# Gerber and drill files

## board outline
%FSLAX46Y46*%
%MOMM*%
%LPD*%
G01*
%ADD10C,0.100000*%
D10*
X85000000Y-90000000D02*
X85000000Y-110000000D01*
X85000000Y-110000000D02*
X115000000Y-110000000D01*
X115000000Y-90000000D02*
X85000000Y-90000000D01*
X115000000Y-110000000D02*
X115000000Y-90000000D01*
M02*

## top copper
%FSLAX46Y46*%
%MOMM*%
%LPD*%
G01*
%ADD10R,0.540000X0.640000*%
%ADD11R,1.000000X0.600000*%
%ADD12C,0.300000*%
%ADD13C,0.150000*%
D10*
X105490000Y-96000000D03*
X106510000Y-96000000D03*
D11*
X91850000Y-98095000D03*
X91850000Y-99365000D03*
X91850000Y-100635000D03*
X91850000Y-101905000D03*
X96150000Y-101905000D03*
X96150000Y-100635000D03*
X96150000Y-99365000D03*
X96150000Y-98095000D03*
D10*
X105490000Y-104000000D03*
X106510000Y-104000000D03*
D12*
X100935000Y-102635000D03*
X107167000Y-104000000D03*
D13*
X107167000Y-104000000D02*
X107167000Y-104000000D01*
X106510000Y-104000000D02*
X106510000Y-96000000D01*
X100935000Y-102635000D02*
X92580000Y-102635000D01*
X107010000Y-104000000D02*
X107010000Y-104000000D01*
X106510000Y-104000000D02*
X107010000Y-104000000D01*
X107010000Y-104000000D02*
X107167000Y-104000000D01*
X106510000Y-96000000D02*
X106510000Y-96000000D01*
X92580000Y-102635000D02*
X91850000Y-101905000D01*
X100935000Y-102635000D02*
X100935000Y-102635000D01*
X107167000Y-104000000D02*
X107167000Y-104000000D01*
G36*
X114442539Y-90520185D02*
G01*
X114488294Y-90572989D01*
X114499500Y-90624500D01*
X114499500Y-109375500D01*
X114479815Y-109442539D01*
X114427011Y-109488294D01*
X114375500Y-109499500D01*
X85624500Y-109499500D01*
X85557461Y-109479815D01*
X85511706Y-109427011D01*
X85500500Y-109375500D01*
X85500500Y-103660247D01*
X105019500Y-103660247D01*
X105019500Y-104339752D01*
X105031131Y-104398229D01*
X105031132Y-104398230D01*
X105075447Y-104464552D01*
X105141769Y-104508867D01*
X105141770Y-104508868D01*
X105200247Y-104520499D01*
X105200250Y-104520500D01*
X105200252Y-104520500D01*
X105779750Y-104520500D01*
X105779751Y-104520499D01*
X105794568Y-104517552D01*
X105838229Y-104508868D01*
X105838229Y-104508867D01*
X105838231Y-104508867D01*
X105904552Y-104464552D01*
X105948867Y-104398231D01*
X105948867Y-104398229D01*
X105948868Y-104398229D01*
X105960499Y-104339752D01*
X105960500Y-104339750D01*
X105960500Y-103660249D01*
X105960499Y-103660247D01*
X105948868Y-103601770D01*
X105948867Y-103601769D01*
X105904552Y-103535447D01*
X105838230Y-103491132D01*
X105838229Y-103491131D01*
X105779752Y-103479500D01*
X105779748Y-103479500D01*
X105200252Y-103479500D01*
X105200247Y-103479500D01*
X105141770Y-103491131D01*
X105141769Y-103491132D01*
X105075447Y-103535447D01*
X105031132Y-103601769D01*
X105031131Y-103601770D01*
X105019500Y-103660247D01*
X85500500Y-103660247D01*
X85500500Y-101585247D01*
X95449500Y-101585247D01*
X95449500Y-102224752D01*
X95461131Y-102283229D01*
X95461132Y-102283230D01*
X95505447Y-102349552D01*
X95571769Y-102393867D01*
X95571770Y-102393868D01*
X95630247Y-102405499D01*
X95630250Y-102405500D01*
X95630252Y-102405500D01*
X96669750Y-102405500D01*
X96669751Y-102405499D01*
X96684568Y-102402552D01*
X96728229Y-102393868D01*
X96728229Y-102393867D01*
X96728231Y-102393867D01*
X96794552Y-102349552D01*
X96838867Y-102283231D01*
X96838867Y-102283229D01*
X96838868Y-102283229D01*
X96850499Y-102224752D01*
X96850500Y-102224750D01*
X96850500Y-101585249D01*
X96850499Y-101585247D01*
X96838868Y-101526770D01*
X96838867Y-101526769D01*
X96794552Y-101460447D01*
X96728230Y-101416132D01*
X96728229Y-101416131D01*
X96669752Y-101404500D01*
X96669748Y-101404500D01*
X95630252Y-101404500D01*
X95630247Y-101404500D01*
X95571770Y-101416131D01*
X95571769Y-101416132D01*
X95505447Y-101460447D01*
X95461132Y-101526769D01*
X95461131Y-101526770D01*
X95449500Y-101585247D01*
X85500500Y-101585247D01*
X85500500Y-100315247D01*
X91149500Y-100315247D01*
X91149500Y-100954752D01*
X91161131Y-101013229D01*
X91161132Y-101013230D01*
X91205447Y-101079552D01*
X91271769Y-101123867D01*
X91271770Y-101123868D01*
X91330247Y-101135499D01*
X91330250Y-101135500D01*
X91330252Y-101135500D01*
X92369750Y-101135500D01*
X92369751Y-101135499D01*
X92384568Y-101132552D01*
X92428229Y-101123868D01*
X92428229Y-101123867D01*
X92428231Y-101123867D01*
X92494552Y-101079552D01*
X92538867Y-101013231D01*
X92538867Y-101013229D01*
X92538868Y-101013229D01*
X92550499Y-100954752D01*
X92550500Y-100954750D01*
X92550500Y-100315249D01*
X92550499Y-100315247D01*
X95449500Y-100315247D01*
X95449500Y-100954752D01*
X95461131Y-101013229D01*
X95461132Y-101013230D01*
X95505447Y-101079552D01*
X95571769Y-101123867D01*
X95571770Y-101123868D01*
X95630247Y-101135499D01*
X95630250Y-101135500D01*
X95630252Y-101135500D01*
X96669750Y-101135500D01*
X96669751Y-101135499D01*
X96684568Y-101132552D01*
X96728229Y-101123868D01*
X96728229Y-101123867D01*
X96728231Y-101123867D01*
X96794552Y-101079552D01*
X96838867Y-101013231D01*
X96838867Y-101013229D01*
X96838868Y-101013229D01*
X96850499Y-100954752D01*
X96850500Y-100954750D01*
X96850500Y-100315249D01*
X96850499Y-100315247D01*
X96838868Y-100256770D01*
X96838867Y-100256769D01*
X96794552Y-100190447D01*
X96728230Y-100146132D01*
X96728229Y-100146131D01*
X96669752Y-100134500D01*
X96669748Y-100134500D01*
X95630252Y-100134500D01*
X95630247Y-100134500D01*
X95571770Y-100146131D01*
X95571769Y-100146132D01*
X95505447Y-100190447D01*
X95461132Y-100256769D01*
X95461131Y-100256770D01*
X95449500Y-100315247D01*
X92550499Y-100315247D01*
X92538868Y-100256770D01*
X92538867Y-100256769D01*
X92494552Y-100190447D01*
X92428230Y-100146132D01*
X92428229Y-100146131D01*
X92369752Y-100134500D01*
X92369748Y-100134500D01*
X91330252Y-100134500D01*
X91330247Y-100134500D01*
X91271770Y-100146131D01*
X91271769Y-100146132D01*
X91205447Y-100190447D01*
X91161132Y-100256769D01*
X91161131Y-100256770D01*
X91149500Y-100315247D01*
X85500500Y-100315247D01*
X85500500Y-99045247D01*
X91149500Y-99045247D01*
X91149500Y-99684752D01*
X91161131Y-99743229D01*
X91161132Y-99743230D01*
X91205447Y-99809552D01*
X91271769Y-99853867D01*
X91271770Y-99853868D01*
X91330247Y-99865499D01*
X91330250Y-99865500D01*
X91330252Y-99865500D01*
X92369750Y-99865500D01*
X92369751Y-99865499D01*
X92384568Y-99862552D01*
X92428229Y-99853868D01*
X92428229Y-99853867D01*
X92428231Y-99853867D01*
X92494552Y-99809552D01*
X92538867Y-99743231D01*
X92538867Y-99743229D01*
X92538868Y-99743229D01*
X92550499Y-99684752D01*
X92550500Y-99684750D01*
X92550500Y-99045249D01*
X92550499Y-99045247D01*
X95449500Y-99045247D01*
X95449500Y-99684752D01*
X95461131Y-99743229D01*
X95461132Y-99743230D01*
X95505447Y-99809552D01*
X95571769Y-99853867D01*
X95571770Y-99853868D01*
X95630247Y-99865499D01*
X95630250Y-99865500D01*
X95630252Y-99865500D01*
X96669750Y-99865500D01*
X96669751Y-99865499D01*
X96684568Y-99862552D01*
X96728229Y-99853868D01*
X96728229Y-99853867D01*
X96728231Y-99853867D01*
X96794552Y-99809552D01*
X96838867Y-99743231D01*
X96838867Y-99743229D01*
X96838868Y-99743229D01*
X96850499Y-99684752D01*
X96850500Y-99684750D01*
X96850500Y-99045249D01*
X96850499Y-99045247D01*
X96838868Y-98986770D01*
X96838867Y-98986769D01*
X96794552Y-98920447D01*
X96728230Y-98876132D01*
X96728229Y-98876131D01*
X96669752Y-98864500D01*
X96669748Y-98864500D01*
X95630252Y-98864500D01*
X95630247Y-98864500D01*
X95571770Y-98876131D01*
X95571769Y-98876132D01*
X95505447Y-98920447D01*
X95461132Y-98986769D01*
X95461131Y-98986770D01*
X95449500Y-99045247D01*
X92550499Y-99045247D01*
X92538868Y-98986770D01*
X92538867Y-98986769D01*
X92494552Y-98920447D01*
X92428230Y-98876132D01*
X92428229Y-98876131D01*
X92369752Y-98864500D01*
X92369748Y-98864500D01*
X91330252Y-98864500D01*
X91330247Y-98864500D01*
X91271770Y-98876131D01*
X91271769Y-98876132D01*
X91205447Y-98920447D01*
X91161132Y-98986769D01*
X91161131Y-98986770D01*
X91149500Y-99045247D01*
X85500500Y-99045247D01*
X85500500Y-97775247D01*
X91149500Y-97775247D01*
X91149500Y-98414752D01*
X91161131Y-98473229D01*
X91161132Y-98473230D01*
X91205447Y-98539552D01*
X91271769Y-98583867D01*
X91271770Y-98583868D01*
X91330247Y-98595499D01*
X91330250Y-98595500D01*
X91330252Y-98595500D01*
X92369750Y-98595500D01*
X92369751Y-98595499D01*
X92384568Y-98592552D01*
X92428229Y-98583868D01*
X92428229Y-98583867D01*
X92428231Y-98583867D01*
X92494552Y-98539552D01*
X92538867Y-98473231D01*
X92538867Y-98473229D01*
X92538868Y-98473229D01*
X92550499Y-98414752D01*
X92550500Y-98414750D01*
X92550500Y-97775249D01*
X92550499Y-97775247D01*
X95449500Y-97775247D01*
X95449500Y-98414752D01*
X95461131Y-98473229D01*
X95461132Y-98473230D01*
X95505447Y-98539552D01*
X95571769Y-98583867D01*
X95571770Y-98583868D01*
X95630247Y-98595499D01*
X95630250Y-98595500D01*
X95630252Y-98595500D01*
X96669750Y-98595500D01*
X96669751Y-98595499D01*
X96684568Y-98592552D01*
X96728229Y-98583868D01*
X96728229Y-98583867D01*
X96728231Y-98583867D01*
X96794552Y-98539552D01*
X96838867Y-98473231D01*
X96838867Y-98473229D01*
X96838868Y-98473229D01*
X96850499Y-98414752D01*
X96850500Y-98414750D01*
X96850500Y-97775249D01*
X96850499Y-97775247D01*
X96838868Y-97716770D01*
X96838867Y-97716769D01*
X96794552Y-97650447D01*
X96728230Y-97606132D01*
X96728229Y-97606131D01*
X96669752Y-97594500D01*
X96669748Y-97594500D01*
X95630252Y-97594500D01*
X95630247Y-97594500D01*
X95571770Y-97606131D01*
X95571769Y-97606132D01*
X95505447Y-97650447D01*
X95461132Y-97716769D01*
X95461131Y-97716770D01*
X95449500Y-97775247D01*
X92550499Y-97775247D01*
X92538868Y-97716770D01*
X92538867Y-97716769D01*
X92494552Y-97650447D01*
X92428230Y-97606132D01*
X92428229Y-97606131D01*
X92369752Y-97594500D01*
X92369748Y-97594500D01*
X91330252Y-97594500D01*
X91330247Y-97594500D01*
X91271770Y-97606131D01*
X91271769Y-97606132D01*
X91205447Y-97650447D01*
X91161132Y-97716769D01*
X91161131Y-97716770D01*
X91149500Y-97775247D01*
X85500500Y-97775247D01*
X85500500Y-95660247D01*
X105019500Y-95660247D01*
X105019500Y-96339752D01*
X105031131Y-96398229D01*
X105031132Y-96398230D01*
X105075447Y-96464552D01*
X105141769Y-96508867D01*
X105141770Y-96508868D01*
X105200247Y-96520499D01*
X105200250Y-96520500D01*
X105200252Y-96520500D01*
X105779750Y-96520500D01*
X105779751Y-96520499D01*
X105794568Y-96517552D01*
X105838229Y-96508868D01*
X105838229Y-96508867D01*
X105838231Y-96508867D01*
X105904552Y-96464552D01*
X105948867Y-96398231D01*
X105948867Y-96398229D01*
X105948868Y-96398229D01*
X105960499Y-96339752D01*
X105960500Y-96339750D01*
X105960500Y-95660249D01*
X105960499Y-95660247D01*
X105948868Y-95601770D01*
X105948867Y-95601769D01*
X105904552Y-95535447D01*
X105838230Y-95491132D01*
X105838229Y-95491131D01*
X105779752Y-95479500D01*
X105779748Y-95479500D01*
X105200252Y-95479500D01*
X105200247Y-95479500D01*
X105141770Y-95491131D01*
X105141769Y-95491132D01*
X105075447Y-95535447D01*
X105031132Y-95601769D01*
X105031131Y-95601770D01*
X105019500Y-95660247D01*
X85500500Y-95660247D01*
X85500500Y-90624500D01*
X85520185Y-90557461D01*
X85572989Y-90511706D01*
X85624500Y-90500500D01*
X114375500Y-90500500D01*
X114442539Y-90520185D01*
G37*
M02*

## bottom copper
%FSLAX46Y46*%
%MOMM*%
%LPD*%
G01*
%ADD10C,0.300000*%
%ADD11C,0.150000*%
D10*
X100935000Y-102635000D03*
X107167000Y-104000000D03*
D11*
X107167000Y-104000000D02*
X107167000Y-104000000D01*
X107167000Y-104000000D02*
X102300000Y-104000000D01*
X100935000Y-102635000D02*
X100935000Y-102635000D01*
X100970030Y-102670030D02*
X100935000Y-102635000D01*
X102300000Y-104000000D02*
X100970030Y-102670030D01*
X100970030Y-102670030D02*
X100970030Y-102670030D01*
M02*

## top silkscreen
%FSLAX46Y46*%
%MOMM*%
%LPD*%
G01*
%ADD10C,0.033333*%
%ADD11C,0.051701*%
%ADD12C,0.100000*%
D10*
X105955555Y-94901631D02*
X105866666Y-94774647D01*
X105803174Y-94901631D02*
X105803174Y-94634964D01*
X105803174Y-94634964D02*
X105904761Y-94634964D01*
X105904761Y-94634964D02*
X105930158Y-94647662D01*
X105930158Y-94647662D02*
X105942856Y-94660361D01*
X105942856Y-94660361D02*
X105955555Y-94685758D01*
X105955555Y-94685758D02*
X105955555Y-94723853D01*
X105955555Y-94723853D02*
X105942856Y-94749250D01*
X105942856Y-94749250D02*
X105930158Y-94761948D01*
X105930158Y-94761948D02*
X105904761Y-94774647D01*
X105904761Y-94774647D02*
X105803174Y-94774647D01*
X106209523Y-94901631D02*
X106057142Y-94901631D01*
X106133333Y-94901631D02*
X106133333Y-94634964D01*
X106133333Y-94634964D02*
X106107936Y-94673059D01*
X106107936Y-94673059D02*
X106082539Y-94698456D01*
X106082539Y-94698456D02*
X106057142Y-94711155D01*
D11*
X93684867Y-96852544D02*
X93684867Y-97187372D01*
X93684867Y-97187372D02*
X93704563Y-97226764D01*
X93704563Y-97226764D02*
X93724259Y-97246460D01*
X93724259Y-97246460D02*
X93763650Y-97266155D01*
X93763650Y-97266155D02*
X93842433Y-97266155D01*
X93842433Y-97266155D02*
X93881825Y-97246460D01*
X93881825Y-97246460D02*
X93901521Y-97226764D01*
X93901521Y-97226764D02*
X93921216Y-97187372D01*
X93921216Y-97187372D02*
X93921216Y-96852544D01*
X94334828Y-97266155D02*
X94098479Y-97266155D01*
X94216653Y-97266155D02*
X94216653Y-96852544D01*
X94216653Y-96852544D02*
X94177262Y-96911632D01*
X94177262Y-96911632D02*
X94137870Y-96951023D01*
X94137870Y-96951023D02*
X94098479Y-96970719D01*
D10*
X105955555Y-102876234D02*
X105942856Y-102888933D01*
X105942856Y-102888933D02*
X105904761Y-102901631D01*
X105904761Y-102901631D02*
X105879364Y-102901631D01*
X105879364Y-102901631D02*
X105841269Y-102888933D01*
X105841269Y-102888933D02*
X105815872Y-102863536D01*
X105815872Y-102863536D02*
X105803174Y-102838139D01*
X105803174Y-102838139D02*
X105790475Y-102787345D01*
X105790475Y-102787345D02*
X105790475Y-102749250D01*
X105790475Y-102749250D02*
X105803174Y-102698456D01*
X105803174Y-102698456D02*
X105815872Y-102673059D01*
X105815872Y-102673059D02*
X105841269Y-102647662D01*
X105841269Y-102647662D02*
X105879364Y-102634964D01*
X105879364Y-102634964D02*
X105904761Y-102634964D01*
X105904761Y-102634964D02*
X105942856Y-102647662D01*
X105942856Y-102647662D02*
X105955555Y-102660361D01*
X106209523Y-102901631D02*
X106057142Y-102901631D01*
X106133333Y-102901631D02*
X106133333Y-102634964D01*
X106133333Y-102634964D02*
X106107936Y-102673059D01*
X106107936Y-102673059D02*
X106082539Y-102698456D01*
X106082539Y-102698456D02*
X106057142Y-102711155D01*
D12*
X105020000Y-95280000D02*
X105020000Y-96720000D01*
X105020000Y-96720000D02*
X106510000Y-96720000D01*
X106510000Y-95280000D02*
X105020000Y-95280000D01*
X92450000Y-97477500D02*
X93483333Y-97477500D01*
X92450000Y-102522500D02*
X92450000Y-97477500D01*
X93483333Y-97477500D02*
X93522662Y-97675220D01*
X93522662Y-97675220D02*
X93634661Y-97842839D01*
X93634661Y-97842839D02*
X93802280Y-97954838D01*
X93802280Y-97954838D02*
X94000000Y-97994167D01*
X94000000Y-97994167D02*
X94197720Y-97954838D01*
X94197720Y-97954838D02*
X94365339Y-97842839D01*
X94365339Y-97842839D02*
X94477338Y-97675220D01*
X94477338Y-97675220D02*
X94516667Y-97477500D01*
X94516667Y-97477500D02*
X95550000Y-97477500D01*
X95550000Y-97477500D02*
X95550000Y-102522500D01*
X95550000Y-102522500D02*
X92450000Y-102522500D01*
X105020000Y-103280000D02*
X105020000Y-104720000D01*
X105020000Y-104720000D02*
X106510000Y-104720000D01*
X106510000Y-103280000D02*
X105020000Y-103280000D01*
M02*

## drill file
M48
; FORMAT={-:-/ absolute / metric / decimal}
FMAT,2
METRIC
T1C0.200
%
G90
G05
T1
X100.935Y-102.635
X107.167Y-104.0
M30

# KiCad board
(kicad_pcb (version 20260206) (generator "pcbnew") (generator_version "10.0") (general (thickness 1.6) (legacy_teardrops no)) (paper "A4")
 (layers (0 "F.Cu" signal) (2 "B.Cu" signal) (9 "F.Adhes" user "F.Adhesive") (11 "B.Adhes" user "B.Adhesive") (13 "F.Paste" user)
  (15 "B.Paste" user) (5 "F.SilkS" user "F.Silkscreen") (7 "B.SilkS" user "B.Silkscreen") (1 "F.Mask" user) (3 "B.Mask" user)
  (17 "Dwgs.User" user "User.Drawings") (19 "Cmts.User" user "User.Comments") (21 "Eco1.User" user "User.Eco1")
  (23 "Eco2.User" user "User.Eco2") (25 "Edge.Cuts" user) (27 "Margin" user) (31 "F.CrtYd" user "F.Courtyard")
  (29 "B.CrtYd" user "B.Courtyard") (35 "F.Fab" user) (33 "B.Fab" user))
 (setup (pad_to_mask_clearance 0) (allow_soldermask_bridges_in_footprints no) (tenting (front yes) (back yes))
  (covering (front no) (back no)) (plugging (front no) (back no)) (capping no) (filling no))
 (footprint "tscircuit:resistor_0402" (layer "F.Cu") (at 106 96)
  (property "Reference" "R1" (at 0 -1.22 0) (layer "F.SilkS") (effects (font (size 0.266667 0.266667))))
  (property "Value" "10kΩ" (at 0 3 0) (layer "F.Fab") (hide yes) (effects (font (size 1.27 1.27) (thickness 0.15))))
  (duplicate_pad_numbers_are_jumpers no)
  (fp_line (start -0.98 -0.72) (end -0.98 0.72) (stroke (width 0.1) (type default)) (layer "F.SilkS"))
  (fp_line (start -0.98 0.72) (end 0.51 0.72) (stroke (width 0.1) (type default)) (layer "F.SilkS"))
  (fp_line (start 0.51 -0.72) (end -0.98 -0.72) (stroke (width 0.1) (type default)) (layer "F.SilkS"))
  (pad "1" smd rect (at -0.51 0) (size 0.54 0.64) (layers "F.Cu" "F.Mask" "F.Paste"))
  (pad "2" smd rect (at 0.51 0) (size 0.54 0.64) (layers "F.Cu" "F.Mask" "F.Paste") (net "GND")))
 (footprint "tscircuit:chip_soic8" (layer "F.Cu") (at 94 100)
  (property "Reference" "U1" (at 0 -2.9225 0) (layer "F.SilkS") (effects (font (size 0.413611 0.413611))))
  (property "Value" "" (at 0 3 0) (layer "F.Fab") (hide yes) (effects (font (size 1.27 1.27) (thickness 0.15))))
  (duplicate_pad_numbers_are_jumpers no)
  (fp_line (start -1.55 -2.5225) (end -0.516667 -2.5225) (stroke (width 0.1) (type default)) (layer "F.SilkS"))
  (fp_line (start -1.55 2.5225) (end -1.55 -2.5225) (stroke (width 0.1) (type default)) (layer "F.SilkS"))
  (fp_line (start -0.516667 -2.5225) (end -0.477338 -2.32478) (stroke (width 0.1) (type default)) (layer "F.SilkS"))
  (fp_line (start -0.477338 -2.32478) (end -0.365339 -2.157161) (stroke (width 0.1) (type default)) (layer "F.SilkS"))
  (fp_line (start -0.365339 -2.157161) (end -0.19772 -2.045162) (stroke (width 0.1) (type default)) (layer "F.SilkS"))
  (fp_line (start -0.19772 -2.045162) (end 0 -2.005833) (stroke (width 0.1) (type default)) (layer "F.SilkS"))
  (fp_line (start 0 -2.005833) (end 0.19772 -2.045162) (stroke (width 0.1) (type default)) (layer "F.SilkS"))
  (fp_line (start 0.19772 -2.045162) (end 0.365339 -2.157161) (stroke (width 0.1) (type default)) (layer "F.SilkS"))
  (fp_line (start 0.365339 -2.157161) (end 0.477338 -2.32478) (stroke (width 0.1) (type default)) (layer "F.SilkS"))
  (fp_line (start 0.477338 -2.32478) (end 0.516667 -2.5225) (stroke (width 0.1) (type default)) (layer "F.SilkS"))
  (fp_line (start 0.516667 -2.5225) (end 1.55 -2.5225) (stroke (width 0.1) (type default)) (layer "F.SilkS"))
  (fp_line (start 1.55 -2.5225) (end 1.55 2.5225) (stroke (width 0.1) (type default)) (layer "F.SilkS"))
  (fp_line (start 1.55 2.5225) (end -1.55 2.5225) (stroke (width 0.1) (type default)) (layer "F.SilkS"))
  (pad "1" smd rect (at -2.15 -1.905) (size 1 0.6) (layers "F.Cu" "F.Mask" "F.Paste"))
  (pad "2" smd rect (at -2.15 -0.635) (size 1 0.6) (layers "F.Cu" "F.Mask" "F.Paste"))
  (pad "3" smd rect (at -2.15 0.635) (size 1 0.6) (layers "F.Cu" "F.Mask" "F.Paste"))
  (pad "4" smd rect (at -2.15 1.905) (size 1 0.6) (layers "F.Cu" "F.Mask" "F.Paste") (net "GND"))
  (pad "5" smd rect (at 2.15 1.905) (size 1 0.6) (layers "F.Cu" "F.Mask" "F.Paste"))
  (pad "6" smd rect (at 2.15 0.635) (size 1 0.6) (layers "F.Cu" "F.Mask" "F.Paste"))
  (pad "7" smd rect (at 2.15 -0.635) (size 1 0.6) (layers "F.Cu" "F.Mask" "F.Paste"))
  (pad "8" smd rect (at 2.15 -1.905) (size 1 0.6) (layers "F.Cu" "F.Mask" "F.Paste")))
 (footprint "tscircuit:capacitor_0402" (layer "F.Cu") (at 106 104)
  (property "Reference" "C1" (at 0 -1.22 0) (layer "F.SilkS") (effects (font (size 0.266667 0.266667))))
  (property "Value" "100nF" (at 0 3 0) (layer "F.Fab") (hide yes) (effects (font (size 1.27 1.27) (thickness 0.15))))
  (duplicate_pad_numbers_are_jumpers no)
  (fp_line (start -0.98 -0.72) (end -0.98 0.72) (stroke (width 0.1) (type default)) (layer "F.SilkS"))
  (fp_line (start -0.98 0.72) (end 0.51 0.72) (stroke (width 0.1) (type default)) (layer "F.SilkS"))
  (fp_line (start 0.51 -0.72) (end -0.98 -0.72) (stroke (width 0.1) (type default)) (layer "F.SilkS"))
  (pad "1" smd rect (at -0.51 0) (size 0.54 0.64) (layers "F.Cu" "F.Mask" "F.Paste"))
  (pad "2" smd rect (at 0.51 0) (size 0.54 0.64) (layers "F.Cu" "F.Mask" "F.Paste") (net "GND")))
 (gr_line (start 85 90) (end 85 110) (stroke (width 0.1) (type solid)) (layer "Edge.Cuts"))
 (gr_line (start 85 110) (end 115 110) (stroke (width 0.1) (type solid)) (layer "Edge.Cuts"))
 (gr_line (start 115 90) (end 85 90) (stroke (width 0.1) (type solid)) (layer "Edge.Cuts"))
 (gr_line (start 115 110) (end 115 90) (stroke (width 0.1) (type solid)) (layer "Edge.Cuts"))
 (segment (start 107.167 104) (end 107.167 104) (width 0.15) (layer "F.Cu") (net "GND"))
 (segment (start 106.51 104) (end 106.51 96) (width 0.15) (layer "F.Cu") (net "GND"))
 (segment (start 100.935 102.635) (end 92.58 102.635) (width 0.15) (layer "F.Cu") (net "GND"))
 (segment (start 107.01 104) (end 107.01 104) (width 0.15) (layer "F.Cu") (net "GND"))
 (segment (start 106.51 104) (end 107.01 104) (width 0.15) (layer "F.Cu") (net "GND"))
 (segment (start 107.01 104) (end 107.167 104) (width 0.15) (layer "F.Cu") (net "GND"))
 (segment (start 106.51 96) (end 106.51 96) (width 0.15) (layer "F.Cu") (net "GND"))
 (segment (start 92.58 102.635) (end 91.85 101.905) (width 0.15) (layer "F.Cu") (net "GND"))
 (segment (start 100.935 102.635) (end 100.935 102.635) (width 0.15) (layer "F.Cu") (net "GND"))
 (segment (start 107.167 104) (end 107.167 104) (width 0.15) (layer "F.Cu") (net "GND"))
 (via (at 100.935 102.635) (size 0.3) (drill 0.2) (layers "F.Cu" "B.Cu") (capping no) (covering (front no) (back no))
  (plugging (front no) (back no)) (filling no) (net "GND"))
 (via (at 107.167 104) (size 0.3) (drill 0.2) (layers "F.Cu" "B.Cu") (capping no) (covering (front no) (back no))
  (plugging (front no) (back no)) (filling no) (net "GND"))
 (segment (start 107.167 104) (end 107.167 104) (width 0.15) (layer "B.Cu") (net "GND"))
 (segment (start 107.167 104) (end 102.3 104) (width 0.15) (layer "B.Cu") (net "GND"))
 (segment (start 100.935 102.635) (end 100.935 102.635) (width 0.15) (layer "B.Cu") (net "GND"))
 (segment (start 100.97003 102.67003) (end 100.935 102.635) (width 0.15) (layer "B.Cu") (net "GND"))
 (segment (start 102.3 104) (end 100.97003 102.67003) (width 0.15) (layer "B.Cu") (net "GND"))
 (segment (start 100.97003 102.67003) (end 100.97003 102.67003) (width 0.15) (layer "B.Cu") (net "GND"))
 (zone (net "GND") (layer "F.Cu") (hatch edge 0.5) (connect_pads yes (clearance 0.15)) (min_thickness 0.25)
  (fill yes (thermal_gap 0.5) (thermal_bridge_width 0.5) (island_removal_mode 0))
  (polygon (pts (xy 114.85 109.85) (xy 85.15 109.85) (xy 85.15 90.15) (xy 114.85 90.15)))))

